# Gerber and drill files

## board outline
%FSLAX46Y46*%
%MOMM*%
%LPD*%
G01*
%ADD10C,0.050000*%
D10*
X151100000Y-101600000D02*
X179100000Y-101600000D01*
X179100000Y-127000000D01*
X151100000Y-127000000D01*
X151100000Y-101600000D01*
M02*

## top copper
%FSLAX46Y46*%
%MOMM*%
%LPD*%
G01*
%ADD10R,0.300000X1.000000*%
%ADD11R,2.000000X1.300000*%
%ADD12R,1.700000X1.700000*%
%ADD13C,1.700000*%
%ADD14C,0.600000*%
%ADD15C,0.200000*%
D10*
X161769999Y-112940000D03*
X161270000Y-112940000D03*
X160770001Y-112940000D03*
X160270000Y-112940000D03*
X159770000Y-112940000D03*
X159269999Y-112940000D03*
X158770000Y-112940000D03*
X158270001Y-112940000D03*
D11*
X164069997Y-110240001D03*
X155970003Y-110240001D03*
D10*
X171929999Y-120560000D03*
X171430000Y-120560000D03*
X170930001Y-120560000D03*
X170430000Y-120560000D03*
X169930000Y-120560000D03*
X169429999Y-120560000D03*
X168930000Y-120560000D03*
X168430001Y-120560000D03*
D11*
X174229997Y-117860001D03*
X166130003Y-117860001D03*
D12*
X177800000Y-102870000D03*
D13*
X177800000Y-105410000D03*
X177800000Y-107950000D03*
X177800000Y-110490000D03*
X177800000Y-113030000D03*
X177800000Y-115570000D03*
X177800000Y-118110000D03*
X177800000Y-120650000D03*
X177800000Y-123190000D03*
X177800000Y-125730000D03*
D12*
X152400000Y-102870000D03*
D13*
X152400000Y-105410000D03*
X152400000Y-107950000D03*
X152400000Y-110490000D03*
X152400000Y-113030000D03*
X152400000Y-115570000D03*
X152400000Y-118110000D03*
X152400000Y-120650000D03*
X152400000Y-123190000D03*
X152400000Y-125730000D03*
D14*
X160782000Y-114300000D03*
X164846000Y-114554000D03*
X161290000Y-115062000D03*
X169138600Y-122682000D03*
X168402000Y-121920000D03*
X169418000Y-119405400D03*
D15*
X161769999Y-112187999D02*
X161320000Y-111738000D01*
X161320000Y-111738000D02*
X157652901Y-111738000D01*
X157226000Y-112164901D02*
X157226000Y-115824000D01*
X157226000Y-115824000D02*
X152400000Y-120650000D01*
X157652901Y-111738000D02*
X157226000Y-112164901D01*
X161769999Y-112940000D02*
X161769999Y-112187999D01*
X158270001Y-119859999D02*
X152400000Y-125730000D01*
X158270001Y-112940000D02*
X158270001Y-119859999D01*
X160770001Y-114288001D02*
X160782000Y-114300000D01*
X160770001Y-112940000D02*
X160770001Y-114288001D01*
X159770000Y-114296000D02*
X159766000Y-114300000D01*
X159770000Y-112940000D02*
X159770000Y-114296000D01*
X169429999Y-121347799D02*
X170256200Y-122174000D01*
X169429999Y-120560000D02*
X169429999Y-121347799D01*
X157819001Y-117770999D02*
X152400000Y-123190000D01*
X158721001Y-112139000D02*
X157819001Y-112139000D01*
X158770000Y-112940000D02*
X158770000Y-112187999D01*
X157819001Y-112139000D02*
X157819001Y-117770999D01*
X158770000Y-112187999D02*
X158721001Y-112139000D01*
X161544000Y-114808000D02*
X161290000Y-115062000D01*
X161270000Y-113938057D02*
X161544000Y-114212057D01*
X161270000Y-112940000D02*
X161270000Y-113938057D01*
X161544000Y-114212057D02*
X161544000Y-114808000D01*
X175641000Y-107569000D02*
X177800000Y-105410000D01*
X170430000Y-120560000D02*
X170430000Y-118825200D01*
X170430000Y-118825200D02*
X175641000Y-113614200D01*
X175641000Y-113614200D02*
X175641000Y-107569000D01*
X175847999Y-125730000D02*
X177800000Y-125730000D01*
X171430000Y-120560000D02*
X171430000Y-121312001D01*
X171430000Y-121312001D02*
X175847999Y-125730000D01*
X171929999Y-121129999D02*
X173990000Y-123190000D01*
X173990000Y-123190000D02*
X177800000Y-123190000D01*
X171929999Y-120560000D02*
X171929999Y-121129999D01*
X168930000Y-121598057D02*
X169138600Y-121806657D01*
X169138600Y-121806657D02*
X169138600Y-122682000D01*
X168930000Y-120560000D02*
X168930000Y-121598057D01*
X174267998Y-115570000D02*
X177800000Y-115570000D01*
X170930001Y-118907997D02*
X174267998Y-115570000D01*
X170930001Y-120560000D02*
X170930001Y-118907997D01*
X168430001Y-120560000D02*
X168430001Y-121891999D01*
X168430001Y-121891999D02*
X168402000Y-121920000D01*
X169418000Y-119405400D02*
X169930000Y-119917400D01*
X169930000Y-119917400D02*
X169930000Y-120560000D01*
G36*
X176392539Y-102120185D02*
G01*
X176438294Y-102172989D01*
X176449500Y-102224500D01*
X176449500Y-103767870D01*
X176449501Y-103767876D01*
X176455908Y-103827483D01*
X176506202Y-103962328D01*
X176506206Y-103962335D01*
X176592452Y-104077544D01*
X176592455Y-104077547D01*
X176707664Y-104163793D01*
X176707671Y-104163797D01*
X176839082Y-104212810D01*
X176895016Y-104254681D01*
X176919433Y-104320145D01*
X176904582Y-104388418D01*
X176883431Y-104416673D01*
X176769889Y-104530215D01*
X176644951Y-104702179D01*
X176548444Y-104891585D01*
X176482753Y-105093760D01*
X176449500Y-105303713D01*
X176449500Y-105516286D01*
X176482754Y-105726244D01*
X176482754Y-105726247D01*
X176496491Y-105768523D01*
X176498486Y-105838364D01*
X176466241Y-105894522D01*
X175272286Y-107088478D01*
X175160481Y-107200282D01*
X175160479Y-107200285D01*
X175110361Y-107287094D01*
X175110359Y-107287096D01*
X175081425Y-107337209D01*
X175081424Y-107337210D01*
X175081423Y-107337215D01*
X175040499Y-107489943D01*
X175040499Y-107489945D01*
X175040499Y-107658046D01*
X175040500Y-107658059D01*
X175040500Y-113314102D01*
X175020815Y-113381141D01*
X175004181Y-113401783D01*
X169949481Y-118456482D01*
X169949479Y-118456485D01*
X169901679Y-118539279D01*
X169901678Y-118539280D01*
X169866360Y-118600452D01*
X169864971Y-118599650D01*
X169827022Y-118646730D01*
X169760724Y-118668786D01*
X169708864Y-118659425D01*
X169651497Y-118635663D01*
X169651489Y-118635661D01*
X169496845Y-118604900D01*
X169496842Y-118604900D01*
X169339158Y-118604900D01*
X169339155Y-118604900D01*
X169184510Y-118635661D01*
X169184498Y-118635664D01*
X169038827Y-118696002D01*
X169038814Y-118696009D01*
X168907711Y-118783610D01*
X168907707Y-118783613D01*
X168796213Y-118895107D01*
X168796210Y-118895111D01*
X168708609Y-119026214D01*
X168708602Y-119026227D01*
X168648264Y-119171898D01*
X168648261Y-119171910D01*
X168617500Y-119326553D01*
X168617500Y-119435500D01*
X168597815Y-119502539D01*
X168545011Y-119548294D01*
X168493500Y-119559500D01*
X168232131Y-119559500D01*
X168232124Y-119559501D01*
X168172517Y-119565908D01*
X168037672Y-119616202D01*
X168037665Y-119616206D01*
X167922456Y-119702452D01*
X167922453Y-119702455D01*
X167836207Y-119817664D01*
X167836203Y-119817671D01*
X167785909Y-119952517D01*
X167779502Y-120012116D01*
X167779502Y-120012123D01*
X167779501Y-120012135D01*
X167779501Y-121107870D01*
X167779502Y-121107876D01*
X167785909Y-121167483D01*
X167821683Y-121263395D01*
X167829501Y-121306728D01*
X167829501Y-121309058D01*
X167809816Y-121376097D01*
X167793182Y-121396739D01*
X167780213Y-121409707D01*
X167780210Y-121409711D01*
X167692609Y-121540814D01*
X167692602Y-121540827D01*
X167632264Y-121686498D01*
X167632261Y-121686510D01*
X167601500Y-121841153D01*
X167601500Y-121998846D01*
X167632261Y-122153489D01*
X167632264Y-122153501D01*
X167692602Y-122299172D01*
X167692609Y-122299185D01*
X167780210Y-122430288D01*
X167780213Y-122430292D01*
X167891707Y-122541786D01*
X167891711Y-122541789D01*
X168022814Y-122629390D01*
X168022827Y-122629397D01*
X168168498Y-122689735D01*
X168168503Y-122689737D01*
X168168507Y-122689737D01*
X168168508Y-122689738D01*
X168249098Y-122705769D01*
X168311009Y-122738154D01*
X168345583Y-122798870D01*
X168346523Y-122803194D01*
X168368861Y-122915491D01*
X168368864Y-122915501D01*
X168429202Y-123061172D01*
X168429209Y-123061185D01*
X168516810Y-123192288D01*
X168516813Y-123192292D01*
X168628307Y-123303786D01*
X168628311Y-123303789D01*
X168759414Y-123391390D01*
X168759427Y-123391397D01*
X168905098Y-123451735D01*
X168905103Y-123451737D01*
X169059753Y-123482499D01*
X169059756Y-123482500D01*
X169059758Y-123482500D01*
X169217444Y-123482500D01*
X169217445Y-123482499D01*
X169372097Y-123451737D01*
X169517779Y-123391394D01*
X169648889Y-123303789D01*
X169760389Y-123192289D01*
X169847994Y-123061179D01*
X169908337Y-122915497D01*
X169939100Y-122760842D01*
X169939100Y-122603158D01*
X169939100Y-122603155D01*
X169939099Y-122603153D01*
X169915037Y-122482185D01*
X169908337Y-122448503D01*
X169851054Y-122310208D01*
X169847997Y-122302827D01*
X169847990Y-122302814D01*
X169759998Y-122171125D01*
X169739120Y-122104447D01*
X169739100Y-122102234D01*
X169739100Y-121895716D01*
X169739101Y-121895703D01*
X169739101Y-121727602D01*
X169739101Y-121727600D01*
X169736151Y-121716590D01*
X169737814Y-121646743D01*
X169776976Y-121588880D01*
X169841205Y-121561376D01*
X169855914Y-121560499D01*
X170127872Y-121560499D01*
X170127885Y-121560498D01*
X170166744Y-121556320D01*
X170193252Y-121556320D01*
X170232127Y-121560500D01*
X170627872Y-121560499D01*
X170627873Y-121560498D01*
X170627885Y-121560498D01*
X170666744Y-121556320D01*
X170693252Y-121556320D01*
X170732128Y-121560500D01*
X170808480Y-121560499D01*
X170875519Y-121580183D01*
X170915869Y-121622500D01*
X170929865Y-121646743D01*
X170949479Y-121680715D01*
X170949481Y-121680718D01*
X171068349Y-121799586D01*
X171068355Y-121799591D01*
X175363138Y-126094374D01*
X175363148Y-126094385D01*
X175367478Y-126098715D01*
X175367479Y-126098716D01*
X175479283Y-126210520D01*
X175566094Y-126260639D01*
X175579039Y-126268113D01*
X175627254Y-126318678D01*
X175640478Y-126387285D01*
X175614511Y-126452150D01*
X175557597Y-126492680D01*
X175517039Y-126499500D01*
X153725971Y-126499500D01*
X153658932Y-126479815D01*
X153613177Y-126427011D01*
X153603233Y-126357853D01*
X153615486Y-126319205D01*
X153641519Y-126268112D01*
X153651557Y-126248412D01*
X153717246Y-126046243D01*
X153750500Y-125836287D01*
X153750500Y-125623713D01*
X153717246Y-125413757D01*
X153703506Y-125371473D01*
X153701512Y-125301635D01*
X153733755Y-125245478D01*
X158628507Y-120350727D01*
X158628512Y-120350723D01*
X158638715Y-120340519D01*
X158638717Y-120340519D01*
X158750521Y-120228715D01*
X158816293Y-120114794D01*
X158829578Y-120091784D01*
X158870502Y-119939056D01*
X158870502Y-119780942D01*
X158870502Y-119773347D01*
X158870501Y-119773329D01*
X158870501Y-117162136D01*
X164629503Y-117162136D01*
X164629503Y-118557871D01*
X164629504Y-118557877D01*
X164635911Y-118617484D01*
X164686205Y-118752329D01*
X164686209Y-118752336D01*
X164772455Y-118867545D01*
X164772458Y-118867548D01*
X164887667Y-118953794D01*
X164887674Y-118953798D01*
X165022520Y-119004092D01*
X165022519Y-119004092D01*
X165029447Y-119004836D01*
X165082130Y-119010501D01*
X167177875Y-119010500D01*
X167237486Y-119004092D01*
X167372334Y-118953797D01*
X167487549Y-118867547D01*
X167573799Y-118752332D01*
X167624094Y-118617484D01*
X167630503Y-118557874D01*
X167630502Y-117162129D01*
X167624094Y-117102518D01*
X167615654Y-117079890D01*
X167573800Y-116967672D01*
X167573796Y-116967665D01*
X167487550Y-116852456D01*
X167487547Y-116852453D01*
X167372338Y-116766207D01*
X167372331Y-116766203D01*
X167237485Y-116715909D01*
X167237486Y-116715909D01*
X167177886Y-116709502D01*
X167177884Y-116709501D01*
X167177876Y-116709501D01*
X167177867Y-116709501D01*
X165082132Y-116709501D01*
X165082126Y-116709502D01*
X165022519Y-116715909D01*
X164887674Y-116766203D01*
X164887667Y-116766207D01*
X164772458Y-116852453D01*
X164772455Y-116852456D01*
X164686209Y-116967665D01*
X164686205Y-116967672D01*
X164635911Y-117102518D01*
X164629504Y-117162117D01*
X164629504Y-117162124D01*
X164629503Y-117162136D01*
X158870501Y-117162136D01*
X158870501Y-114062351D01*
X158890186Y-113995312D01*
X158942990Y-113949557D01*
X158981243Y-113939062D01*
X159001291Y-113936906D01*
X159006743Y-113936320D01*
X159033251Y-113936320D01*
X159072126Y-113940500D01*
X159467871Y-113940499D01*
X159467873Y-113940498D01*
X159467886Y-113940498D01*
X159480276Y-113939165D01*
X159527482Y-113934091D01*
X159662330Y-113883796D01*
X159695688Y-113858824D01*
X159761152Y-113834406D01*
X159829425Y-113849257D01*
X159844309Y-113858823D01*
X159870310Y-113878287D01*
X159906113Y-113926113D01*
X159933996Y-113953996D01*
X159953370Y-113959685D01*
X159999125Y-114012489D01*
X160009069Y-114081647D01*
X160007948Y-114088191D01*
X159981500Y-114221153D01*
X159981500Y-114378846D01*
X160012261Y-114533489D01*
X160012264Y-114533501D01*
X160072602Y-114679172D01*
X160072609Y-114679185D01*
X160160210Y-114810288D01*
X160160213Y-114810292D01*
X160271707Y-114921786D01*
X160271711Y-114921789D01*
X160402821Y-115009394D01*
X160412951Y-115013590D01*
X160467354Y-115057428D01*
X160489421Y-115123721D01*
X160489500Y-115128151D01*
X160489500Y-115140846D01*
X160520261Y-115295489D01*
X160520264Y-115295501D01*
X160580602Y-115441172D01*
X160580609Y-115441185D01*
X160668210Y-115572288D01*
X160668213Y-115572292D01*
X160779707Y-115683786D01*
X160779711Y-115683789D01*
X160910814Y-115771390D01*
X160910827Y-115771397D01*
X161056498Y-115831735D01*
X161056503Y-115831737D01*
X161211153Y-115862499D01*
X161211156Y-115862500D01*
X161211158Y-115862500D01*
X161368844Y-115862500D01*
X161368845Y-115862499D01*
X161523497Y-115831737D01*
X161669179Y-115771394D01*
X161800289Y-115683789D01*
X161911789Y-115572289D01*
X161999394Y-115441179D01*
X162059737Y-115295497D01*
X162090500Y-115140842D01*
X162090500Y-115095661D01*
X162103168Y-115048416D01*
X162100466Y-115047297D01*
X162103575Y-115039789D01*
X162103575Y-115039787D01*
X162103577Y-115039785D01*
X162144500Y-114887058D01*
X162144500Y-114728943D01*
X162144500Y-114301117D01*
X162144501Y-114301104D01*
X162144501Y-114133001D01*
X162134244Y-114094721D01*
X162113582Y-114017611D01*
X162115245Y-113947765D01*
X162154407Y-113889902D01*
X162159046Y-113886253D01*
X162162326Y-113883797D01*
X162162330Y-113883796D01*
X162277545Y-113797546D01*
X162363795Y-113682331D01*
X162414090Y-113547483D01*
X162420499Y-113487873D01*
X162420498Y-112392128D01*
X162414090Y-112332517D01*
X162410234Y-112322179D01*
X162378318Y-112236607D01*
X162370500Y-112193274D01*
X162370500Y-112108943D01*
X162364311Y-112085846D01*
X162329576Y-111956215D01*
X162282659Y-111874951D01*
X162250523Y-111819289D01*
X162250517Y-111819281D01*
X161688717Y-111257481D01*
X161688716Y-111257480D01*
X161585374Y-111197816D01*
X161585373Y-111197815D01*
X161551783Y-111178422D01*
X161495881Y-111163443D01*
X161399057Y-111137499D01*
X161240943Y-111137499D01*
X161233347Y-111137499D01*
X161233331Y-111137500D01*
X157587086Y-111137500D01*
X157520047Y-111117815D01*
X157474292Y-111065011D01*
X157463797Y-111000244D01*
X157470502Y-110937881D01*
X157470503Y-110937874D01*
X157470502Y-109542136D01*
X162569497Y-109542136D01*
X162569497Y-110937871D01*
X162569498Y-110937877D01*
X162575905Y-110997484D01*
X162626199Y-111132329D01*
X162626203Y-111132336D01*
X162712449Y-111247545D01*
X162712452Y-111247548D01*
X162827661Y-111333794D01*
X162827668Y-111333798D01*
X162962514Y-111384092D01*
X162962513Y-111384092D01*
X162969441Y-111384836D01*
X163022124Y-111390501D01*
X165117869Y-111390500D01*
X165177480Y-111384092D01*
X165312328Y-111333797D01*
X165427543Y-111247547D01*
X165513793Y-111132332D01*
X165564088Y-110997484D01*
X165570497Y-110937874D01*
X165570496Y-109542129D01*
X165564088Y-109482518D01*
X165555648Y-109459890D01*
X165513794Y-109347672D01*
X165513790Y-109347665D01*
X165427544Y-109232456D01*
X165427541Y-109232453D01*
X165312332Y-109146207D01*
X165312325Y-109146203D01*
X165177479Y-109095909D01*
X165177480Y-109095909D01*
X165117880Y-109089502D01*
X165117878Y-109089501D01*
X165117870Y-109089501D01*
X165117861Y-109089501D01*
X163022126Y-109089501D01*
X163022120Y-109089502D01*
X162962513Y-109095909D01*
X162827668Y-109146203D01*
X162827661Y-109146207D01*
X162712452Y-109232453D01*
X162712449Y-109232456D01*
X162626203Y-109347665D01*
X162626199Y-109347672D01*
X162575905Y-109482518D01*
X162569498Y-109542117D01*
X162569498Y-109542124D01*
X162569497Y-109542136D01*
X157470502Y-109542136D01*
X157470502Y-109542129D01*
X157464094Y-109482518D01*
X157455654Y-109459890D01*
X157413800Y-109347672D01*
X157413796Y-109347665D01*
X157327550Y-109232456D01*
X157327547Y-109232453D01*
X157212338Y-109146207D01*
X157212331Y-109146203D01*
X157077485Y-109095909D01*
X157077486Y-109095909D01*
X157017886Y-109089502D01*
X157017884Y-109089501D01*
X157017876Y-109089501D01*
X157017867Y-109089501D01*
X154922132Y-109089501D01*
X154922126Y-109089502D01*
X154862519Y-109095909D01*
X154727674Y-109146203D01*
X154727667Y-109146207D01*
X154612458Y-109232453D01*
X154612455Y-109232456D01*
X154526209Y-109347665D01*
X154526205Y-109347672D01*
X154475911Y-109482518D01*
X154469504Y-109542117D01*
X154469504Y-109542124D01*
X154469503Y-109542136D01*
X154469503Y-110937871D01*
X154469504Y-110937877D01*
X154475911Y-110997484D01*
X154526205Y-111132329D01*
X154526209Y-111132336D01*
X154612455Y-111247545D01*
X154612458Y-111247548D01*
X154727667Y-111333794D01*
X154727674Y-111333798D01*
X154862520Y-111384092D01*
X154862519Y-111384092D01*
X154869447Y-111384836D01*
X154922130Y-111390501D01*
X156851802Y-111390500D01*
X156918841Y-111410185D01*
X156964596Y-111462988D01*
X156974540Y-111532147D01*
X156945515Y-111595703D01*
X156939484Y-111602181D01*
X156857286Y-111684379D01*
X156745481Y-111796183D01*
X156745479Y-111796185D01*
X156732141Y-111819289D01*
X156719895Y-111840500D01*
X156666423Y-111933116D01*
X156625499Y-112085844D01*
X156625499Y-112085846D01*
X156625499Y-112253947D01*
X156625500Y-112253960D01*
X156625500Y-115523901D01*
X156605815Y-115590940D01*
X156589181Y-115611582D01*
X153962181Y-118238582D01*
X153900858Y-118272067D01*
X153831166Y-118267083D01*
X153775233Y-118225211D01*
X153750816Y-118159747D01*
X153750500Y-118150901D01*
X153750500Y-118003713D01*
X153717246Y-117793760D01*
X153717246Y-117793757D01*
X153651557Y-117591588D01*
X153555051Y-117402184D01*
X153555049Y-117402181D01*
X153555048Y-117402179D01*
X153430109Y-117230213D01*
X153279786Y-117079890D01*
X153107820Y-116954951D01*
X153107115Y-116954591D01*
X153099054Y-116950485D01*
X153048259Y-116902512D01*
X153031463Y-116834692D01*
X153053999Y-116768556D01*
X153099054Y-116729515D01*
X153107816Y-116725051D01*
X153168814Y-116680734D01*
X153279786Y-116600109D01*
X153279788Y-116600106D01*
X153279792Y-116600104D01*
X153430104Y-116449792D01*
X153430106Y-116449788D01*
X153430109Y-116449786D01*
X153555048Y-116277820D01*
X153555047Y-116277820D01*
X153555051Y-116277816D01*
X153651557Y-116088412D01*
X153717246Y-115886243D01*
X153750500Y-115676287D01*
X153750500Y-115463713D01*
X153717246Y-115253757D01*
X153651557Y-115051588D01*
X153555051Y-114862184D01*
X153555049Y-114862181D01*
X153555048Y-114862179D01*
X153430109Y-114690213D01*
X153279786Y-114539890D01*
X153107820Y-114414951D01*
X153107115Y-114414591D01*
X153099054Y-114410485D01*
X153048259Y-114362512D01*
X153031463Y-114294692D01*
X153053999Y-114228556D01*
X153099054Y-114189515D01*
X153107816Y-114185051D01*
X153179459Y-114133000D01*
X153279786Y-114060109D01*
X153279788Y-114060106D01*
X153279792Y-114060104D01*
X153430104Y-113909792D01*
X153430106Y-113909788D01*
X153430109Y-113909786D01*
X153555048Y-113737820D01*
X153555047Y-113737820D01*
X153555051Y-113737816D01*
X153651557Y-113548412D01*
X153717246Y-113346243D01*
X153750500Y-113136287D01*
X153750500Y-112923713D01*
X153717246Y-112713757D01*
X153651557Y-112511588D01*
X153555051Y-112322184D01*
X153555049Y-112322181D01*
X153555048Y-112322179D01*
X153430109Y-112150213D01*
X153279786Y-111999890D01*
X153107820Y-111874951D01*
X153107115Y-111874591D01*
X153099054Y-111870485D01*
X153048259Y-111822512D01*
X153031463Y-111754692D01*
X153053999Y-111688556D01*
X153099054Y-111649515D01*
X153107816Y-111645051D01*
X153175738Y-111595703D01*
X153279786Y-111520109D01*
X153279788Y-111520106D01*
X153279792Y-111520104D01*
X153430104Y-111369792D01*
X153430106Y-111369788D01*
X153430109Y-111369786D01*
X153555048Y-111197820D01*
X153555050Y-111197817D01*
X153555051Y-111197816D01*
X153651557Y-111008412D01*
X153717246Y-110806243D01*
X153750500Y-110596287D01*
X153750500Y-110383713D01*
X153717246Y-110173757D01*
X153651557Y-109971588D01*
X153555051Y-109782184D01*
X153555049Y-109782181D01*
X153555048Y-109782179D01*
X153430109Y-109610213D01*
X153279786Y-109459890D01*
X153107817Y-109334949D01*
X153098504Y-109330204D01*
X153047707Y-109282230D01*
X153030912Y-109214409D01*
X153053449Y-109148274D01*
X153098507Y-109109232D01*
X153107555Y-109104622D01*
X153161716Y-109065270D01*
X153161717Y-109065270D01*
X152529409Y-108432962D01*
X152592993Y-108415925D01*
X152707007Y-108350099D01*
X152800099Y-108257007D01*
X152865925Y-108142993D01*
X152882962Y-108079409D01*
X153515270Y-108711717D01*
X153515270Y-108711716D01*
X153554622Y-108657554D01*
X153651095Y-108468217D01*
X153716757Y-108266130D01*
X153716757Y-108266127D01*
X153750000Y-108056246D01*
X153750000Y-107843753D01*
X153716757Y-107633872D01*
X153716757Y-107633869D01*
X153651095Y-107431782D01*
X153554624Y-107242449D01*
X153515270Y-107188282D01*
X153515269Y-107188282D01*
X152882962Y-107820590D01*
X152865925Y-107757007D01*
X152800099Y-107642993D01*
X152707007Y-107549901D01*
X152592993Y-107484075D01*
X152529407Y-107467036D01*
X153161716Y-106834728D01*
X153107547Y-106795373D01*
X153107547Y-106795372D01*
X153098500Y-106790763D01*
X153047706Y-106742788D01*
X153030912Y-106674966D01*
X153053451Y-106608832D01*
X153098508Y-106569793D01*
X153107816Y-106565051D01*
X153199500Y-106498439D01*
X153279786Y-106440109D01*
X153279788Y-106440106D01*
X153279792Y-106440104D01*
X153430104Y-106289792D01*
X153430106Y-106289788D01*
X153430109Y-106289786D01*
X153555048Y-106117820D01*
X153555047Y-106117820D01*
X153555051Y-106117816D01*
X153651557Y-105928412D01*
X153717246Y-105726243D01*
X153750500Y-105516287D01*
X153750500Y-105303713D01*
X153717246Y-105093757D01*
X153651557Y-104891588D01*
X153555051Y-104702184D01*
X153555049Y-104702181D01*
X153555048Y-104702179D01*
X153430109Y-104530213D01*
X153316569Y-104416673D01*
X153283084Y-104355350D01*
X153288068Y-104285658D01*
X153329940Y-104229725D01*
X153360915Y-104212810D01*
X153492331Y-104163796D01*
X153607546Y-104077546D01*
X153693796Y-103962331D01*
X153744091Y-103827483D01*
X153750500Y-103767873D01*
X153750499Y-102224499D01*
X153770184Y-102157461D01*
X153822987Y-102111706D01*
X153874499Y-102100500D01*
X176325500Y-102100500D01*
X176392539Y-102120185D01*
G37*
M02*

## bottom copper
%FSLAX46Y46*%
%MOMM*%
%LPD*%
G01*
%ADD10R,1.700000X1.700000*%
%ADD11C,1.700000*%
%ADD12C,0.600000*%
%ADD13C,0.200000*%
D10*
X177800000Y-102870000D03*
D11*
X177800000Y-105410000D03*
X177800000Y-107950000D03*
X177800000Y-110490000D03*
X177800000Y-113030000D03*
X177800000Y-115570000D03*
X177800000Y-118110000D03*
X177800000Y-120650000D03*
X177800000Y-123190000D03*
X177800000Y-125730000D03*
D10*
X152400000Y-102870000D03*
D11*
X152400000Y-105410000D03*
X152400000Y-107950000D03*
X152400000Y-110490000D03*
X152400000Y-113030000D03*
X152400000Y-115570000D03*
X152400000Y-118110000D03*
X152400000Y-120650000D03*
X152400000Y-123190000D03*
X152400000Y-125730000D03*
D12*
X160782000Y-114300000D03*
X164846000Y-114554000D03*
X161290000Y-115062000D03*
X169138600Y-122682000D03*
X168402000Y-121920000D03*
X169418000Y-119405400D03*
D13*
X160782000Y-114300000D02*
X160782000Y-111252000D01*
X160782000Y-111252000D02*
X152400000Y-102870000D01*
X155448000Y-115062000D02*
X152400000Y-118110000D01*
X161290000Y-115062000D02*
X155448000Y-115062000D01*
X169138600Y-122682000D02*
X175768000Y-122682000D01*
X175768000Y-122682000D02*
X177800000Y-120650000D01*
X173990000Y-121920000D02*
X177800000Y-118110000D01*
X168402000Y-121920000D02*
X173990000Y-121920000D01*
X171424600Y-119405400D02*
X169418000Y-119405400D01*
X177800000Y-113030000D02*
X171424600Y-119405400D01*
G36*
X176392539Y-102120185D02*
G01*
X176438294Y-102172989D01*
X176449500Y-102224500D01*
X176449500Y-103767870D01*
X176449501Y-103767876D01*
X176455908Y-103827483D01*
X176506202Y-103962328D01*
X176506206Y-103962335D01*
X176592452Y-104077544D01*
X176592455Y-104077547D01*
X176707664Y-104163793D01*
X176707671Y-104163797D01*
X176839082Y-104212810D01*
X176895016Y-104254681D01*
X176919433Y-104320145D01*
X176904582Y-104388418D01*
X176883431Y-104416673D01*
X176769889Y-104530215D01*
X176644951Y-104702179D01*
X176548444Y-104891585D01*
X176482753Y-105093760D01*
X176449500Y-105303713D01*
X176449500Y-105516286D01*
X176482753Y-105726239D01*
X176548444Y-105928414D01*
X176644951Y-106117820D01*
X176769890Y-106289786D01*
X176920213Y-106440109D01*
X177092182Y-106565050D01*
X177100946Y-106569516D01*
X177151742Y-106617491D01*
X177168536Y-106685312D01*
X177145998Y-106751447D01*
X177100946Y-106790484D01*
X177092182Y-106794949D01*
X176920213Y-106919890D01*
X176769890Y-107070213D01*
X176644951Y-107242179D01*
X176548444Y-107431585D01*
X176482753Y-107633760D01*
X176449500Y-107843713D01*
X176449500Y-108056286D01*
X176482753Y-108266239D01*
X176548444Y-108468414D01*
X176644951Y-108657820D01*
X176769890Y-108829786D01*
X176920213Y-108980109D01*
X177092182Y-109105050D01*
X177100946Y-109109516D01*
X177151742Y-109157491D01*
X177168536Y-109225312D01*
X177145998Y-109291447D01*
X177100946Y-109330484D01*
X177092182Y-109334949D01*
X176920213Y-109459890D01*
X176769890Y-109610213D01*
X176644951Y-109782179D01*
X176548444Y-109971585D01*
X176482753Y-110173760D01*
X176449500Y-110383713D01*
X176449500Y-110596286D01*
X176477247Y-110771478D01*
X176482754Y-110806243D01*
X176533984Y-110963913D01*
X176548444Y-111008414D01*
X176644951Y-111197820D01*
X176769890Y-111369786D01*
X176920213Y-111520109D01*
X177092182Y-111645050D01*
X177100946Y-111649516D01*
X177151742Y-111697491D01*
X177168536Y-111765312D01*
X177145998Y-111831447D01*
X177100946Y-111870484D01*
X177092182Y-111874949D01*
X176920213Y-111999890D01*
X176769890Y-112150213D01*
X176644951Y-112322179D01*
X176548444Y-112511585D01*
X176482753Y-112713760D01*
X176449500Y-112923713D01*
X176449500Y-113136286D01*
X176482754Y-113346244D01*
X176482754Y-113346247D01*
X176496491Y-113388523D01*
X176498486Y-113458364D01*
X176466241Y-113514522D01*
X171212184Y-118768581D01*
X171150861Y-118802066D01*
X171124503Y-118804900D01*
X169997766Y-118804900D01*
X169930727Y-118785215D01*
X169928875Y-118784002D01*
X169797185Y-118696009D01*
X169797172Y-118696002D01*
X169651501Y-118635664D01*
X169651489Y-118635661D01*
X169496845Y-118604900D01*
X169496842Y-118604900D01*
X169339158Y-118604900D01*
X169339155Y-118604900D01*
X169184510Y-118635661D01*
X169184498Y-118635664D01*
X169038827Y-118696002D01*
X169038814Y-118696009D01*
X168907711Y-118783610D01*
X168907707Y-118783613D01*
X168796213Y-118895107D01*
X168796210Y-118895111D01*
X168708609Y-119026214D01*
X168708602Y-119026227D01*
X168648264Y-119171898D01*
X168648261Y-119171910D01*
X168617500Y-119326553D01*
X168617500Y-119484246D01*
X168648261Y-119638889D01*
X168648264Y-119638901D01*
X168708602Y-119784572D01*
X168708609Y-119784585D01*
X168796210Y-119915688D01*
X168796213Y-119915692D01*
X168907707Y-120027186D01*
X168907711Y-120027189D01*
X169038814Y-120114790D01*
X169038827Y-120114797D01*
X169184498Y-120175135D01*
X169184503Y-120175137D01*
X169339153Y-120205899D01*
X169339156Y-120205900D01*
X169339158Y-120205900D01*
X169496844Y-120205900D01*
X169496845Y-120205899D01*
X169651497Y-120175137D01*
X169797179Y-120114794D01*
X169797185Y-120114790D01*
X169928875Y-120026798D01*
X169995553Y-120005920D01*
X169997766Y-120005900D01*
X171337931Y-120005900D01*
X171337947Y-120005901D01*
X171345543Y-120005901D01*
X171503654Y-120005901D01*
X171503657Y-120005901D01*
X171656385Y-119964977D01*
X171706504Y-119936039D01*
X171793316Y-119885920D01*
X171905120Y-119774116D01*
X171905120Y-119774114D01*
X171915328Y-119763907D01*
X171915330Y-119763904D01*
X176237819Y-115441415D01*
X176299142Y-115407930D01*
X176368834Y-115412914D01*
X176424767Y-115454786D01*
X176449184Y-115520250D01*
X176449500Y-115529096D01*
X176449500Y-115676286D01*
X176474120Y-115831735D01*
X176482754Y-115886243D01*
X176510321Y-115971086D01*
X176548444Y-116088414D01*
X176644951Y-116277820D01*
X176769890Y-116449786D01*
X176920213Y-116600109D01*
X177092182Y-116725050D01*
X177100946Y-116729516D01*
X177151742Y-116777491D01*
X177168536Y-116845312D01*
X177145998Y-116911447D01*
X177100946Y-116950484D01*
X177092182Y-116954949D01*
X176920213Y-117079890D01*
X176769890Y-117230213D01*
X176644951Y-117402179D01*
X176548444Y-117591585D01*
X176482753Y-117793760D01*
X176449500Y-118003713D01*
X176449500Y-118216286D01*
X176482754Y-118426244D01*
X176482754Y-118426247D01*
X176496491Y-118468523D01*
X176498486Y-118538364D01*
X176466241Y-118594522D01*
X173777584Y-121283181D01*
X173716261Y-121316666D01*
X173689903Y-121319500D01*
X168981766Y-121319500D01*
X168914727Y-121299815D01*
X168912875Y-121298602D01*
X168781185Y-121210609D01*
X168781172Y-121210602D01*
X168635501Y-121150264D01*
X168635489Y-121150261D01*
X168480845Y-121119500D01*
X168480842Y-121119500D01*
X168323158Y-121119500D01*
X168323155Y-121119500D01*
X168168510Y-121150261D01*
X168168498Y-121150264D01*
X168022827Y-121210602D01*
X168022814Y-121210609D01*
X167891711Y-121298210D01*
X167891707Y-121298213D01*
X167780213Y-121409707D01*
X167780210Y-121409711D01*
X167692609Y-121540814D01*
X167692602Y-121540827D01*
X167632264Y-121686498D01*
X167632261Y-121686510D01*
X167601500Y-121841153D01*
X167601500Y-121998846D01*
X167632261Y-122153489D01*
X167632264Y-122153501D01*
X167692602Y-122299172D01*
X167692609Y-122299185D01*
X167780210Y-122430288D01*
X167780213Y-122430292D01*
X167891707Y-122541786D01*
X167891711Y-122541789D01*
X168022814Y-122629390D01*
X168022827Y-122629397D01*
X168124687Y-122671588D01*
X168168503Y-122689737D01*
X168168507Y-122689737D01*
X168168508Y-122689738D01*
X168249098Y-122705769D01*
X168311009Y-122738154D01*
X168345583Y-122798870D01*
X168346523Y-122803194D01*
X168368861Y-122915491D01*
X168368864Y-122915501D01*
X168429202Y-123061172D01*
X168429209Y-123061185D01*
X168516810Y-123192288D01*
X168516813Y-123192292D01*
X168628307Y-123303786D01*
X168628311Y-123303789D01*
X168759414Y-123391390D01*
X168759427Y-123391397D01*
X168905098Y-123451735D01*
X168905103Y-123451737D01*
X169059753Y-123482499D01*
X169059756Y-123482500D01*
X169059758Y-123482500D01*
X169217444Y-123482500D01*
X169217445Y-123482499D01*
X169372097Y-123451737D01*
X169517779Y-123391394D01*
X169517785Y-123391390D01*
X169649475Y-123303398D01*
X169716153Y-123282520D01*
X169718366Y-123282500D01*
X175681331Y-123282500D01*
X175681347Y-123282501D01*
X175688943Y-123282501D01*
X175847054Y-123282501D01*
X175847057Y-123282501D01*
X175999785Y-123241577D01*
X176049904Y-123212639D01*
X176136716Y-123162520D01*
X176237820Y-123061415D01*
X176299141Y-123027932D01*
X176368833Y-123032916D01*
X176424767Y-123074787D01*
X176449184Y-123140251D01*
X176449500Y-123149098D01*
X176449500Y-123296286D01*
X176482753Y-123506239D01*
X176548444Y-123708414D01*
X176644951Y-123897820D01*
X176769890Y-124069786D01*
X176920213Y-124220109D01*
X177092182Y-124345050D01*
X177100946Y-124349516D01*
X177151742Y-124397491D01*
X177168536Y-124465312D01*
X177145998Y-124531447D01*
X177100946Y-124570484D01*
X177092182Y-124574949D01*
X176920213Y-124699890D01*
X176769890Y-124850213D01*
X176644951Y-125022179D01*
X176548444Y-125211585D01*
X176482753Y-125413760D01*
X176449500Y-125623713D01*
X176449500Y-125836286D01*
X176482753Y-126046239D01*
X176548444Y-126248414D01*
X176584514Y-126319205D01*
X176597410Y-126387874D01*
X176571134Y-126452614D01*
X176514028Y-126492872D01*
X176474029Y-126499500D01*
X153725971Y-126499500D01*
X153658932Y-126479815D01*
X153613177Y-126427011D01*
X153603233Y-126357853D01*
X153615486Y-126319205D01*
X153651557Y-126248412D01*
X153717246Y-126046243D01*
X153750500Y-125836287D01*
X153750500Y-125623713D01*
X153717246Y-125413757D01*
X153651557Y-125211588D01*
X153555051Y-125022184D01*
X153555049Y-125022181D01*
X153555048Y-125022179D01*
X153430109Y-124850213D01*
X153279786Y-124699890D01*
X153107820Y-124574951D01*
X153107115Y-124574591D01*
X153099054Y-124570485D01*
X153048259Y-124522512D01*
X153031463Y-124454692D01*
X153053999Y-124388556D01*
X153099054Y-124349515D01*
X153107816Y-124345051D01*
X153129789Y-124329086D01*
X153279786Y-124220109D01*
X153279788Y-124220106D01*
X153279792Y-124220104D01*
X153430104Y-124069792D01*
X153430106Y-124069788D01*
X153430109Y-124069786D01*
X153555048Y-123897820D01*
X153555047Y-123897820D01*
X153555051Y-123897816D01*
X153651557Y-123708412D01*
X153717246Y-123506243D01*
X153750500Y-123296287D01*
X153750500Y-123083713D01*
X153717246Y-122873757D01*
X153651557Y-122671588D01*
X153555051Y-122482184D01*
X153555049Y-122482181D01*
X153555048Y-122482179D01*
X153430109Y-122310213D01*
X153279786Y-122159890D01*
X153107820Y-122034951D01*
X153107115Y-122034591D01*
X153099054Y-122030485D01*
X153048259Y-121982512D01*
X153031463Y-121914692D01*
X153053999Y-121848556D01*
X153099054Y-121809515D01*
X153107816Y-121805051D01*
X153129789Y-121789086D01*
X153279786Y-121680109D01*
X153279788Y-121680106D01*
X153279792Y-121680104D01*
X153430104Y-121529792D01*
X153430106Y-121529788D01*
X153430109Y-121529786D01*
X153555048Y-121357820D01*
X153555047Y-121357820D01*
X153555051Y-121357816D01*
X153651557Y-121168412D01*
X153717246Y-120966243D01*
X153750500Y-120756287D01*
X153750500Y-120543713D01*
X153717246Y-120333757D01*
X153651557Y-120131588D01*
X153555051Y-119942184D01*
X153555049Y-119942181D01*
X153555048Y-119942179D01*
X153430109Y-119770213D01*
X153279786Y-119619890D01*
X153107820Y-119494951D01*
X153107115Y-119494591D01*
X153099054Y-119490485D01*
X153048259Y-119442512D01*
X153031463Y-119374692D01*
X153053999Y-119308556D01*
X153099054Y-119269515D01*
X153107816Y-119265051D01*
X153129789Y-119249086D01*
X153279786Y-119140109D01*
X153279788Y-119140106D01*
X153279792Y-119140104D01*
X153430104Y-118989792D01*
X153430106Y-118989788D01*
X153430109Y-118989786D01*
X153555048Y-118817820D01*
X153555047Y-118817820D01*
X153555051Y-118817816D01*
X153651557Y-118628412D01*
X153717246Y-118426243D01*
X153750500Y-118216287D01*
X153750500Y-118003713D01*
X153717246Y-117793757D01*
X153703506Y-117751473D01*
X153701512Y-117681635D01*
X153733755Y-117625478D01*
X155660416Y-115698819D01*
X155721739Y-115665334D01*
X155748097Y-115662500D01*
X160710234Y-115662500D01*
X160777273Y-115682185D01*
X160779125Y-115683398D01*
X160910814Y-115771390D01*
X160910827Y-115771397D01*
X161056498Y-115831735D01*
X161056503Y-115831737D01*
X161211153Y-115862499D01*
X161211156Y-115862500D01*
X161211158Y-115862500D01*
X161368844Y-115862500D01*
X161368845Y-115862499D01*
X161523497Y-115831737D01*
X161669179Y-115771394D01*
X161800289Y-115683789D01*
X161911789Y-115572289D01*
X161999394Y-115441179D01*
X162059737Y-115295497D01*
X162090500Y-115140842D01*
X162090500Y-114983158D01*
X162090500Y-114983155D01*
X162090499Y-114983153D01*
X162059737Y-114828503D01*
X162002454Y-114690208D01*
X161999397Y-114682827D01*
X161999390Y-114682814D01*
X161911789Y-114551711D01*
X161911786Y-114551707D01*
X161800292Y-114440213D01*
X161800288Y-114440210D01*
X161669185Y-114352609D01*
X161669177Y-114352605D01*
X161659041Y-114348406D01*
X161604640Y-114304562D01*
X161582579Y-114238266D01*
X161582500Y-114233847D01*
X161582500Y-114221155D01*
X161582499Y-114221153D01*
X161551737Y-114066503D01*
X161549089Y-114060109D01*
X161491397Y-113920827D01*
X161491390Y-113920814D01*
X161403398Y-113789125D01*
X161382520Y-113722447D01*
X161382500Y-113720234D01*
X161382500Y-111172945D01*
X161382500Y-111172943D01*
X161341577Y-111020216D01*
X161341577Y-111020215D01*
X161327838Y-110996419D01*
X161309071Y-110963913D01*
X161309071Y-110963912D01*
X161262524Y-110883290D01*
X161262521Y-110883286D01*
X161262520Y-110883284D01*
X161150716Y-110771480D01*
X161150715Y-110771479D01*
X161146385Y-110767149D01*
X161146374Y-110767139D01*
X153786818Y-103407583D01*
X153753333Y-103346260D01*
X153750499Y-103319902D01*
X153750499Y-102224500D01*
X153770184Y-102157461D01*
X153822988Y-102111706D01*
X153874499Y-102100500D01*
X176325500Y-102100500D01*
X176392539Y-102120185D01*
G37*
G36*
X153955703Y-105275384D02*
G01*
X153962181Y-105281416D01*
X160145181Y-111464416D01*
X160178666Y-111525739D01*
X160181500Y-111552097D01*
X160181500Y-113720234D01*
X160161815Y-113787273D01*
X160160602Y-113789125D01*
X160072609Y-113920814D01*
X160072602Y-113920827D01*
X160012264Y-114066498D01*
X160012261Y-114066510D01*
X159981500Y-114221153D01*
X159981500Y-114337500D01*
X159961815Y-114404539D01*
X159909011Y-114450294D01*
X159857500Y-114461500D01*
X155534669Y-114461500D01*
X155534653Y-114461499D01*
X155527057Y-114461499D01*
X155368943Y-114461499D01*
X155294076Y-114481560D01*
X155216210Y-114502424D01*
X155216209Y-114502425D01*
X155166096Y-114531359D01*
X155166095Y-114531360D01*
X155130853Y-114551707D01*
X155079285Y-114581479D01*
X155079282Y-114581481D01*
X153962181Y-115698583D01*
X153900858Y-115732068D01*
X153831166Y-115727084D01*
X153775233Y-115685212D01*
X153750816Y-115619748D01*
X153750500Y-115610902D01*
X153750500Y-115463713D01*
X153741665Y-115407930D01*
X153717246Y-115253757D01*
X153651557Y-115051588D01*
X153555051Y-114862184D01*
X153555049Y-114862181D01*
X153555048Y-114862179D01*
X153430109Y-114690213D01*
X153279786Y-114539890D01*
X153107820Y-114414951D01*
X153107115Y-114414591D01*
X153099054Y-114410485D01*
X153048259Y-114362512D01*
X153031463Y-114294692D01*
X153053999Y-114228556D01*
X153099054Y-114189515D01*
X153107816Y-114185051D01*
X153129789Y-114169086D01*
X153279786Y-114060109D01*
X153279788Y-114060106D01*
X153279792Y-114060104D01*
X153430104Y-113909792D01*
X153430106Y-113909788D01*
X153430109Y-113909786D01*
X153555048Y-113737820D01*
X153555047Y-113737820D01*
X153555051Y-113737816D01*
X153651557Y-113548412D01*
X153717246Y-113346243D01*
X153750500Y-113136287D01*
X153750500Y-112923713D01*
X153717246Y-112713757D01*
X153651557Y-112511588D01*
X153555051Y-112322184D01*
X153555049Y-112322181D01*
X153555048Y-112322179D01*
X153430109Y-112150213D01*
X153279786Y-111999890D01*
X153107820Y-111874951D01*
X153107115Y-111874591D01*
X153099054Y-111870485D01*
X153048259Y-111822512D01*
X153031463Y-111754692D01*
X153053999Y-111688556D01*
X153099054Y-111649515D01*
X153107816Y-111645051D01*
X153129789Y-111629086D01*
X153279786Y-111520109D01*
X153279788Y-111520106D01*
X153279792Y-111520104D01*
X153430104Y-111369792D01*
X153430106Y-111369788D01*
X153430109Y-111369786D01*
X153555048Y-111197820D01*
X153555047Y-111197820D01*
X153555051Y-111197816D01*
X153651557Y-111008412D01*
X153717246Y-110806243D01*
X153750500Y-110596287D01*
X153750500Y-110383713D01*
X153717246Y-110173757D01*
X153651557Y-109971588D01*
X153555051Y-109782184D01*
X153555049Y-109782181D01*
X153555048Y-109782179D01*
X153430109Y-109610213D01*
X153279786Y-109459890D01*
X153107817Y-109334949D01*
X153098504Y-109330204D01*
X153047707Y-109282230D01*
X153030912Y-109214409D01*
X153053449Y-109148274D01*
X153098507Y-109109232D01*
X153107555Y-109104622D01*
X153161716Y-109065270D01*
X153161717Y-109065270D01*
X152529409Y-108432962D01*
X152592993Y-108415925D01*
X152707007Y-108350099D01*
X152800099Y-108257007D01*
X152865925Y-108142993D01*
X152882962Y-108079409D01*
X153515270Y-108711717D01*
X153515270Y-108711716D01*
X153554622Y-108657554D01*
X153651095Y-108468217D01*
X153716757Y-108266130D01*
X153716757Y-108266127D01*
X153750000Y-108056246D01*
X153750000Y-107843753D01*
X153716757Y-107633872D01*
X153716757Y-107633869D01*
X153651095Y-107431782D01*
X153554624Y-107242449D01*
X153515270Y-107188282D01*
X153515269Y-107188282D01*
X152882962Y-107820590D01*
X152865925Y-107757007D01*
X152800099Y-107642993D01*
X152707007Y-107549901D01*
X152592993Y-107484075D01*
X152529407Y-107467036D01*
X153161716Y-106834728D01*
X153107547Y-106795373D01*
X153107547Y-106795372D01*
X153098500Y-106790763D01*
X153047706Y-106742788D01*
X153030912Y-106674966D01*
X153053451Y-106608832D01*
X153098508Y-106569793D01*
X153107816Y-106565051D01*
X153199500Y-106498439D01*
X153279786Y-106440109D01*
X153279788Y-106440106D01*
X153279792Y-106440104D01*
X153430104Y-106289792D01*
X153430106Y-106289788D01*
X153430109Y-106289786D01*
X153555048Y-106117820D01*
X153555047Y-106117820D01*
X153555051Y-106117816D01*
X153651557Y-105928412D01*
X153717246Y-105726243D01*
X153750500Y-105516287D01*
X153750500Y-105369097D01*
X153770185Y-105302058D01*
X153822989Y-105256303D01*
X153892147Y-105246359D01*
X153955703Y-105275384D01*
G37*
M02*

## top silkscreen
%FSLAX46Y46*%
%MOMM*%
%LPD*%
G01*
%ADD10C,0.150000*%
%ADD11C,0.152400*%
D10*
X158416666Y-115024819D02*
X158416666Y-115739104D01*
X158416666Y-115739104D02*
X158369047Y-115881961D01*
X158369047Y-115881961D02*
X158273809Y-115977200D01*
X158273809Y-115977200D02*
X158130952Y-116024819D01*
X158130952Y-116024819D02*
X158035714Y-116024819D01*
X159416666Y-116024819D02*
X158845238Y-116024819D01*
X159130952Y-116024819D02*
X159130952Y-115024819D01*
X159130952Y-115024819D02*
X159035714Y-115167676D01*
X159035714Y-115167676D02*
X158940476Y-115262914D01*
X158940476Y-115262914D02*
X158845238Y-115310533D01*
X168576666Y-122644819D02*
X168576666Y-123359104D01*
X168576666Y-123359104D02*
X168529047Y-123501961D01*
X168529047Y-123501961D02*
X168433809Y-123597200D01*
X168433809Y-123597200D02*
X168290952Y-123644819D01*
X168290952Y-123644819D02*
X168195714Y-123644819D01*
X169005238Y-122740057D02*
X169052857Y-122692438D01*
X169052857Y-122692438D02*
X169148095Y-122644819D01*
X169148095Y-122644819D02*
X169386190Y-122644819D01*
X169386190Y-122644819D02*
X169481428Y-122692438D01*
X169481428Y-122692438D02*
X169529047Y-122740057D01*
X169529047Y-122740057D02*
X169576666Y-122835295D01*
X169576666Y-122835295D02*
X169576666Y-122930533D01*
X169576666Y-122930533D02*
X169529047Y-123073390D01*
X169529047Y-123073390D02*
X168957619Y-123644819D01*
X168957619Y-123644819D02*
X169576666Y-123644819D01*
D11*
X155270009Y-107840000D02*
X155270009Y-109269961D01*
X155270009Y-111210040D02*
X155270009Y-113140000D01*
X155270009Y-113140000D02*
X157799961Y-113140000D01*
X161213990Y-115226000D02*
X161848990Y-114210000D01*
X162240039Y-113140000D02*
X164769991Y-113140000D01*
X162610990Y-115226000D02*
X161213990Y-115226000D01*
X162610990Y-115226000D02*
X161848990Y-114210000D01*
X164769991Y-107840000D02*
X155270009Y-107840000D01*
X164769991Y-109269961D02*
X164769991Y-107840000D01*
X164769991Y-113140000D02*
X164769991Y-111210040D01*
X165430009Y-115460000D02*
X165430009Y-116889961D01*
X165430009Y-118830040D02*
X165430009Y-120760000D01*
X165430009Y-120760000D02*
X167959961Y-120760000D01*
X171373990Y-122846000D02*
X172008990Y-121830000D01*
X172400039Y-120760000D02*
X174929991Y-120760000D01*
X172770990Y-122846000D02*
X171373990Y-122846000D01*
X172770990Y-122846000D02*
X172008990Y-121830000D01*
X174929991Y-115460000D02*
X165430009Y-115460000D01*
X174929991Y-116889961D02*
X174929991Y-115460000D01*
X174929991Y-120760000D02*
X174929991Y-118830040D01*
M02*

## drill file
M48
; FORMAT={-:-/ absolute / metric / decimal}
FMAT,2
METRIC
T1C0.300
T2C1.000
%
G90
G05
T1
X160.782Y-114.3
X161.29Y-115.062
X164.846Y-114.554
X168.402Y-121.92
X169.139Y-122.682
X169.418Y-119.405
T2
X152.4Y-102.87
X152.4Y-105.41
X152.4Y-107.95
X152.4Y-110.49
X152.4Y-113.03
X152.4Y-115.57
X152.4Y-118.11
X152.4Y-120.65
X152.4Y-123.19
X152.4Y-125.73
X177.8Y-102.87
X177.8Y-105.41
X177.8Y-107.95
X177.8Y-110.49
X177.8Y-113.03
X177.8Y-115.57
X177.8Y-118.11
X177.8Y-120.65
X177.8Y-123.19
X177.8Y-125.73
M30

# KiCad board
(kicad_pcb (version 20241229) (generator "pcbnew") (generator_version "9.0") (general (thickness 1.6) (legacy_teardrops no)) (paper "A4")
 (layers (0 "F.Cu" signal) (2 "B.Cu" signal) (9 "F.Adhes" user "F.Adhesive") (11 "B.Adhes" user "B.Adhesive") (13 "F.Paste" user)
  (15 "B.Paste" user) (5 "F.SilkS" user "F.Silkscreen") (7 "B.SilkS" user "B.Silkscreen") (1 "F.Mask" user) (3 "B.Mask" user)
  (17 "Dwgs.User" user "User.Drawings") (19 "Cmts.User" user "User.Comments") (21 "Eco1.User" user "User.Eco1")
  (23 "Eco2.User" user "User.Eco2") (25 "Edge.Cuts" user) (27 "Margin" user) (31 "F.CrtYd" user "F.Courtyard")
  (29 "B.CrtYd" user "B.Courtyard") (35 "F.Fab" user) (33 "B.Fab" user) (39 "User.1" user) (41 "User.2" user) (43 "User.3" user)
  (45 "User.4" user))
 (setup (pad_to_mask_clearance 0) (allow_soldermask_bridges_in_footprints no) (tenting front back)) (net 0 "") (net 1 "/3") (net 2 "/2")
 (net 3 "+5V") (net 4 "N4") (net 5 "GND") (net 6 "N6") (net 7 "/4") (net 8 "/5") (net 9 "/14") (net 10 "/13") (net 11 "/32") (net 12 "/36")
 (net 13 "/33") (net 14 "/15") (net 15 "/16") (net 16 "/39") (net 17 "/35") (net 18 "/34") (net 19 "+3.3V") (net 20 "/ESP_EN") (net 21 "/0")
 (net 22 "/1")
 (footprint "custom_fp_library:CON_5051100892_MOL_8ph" (layer "F.Cu") (at 160.02 110.49 180)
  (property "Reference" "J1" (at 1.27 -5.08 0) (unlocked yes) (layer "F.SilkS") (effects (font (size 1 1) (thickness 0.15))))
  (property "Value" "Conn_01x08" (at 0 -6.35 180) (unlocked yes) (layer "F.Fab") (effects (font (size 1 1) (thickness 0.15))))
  (fp_line (start 4.749991 2.65) (end 4.749991 1.220039) (stroke (width 0.1524) (type solid)) (layer "F.SilkS"))
  (fp_line (start 4.749991 -0.72004) (end 4.749991 -2.65) (stroke (width 0.1524) (type solid)) (layer "F.SilkS"))
  (fp_line (start 4.749991 -2.65) (end 2.220039 -2.65) (stroke (width 0.1524) (type solid)) (layer "F.SilkS"))
  (fp_line (start -1.19399 -4.736) (end -1.82899 -3.72) (stroke (width 0.1524) (type solid)) (layer "F.SilkS"))
  (fp_line (start -2.220039 -2.65) (end -4.749991 -2.65) (stroke (width 0.1524) (type solid)) (layer "F.SilkS"))
  (fp_line (start -2.59099 -4.736) (end -1.19399 -4.736) (stroke (width 0.1524) (type solid)) (layer "F.SilkS"))
  (fp_line (start -2.59099 -4.736) (end -1.82899 -3.72) (stroke (width 0.1524) (type solid)) (layer "F.SilkS"))
  (fp_line (start -4.749991 2.65) (end 4.749991 2.65) (stroke (width 0.1524) (type solid)) (layer "F.SilkS"))
  (fp_line (start -4.749991 1.220039) (end -4.749991 2.65) (stroke (width 0.1524) (type solid)) (layer "F.SilkS"))
  (fp_line (start -4.749991 -2.65) (end -4.749991 -0.72004) (stroke (width 0.1524) (type solid)) (layer "F.SilkS"))
  (pad "1" smd rect (at -1.749999 -2.45 180) (size 0.3 1) (layers "F.Cu" "F.Mask" "F.Paste") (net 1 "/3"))
  (pad "2" smd rect (at -1.25 -2.45 180) (size 0.3 1) (layers "F.Cu" "F.Mask" "F.Paste") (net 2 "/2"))
  (pad "3" smd rect (at -0.750001 -2.45 180) (size 0.3 1) (layers "F.Cu" "F.Mask" "F.Paste") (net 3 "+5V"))
  (pad "4" smd rect (at -0.25 -2.45 180) (size 0.3 1) (layers "F.Cu" "F.Mask" "F.Paste") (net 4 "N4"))
  (pad "5" smd rect (at 0.25 -2.45 180) (size 0.3 1) (layers "F.Cu" "F.Mask" "F.Paste") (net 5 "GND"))
  (pad "6" smd rect (at 0.750001 -2.45 180) (size 0.3 1) (layers "F.Cu" "F.Mask" "F.Paste") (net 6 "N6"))
  (pad "7" smd rect (at 1.25 -2.45 180) (size 0.3 1) (layers "F.Cu" "F.Mask" "F.Paste") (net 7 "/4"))
  (pad "8" smd rect (at 1.749999 -2.45 180) (size 0.3 1) (layers "F.Cu" "F.Mask" "F.Paste") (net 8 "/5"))
  (pad "P1" smd rect (at -4.049997 0.249999 180) (size 2 1.3) (layers "F.Cu" "F.Mask" "F.Paste"))
  (pad "P2" smd rect (at 4.049997 0.249999 180) (size 2 1.3) (layers "F.Cu" "F.Mask" "F.Paste")))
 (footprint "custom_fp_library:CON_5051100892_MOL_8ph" (layer "F.Cu") (at 170.18 118.11 180)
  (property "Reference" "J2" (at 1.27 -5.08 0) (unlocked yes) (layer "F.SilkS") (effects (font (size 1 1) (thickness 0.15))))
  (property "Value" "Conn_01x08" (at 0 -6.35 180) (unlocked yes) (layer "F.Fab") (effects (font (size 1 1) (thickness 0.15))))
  (fp_line (start 4.749991 2.65) (end 4.749991 1.220039) (stroke (width 0.1524) (type solid)) (layer "F.SilkS"))
  (fp_line (start 4.749991 -0.72004) (end 4.749991 -2.65) (stroke (width 0.1524) (type solid)) (layer "F.SilkS"))
  (fp_line (start 4.749991 -2.65) (end 2.220039 -2.65) (stroke (width 0.1524) (type solid)) (layer "F.SilkS"))
  (fp_line (start -1.19399 -4.736) (end -1.82899 -3.72) (stroke (width 0.1524) (type solid)) (layer "F.SilkS"))
  (fp_line (start -2.220039 -2.65) (end -4.749991 -2.65) (stroke (width 0.1524) (type solid)) (layer "F.SilkS"))
  (fp_line (start -2.59099 -4.736) (end -1.19399 -4.736) (stroke (width 0.1524) (type solid)) (layer "F.SilkS"))
  (fp_line (start -2.59099 -4.736) (end -1.82899 -3.72) (stroke (width 0.1524) (type solid)) (layer "F.SilkS"))
  (fp_line (start -4.749991 2.65) (end 4.749991 2.65) (stroke (width 0.1524) (type solid)) (layer "F.SilkS"))
  (fp_line (start -4.749991 1.220039) (end -4.749991 2.65) (stroke (width 0.1524) (type solid)) (layer "F.SilkS"))
  (fp_line (start -4.749991 -2.65) (end -4.749991 -0.72004) (stroke (width 0.1524) (type solid)) (layer "F.SilkS"))
  (pad "1" smd rect (at -1.749999 -2.45 180) (size 0.3 1) (layers "F.Cu" "F.Mask" "F.Paste") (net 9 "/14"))
  (pad "2" smd rect (at -1.25 -2.45 180) (size 0.3 1) (layers "F.Cu" "F.Mask" "F.Paste") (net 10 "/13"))
  (pad "3" smd rect (at -0.750001 -2.45 180) (size 0.3 1) (layers "F.Cu" "F.Mask" "F.Paste") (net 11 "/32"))
  (pad "4" smd rect (at -0.25 -2.45 180) (size 0.3 1) (layers "F.Cu" "F.Mask" "F.Paste") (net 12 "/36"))
  (pad "5" smd rect (at 0.25 -2.45 180) (size 0.3 1) (layers "F.Cu" "F.Mask" "F.Paste") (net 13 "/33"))
  (pad "6" smd rect (at 0.750001 -2.45 180) (size 0.3 1) (layers "F.Cu" "F.Mask" "F.Paste") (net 5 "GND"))
  (pad "7" smd rect (at 1.25 -2.45 180) (size 0.3 1) (layers "F.Cu" "F.Mask" "F.Paste") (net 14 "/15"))
  (pad "8" smd rect (at 1.749999 -2.45 180) (size 0.3 1) (layers "F.Cu" "F.Mask" "F.Paste") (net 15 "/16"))
  (pad "P1" smd rect (at -4.049997 0.249999 180) (size 2 1.3) (layers "F.Cu" "F.Mask" "F.Paste"))
  (pad "P2" smd rect (at 4.049997 0.249999 180) (size 2 1.3) (layers "F.Cu" "F.Mask" "F.Paste")))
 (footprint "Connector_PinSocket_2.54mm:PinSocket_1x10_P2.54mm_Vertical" (layer "B.Cu") (at 177.8 102.87 180)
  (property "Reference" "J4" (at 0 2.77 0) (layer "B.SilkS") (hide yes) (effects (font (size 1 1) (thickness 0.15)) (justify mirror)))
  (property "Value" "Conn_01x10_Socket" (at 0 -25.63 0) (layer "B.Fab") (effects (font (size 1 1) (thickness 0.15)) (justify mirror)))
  (pad "1" thru_hole rect (at 0 0 180) (size 1.7 1.7) (drill 1) (layers "*.Cu" "*.Mask") (remove_unused_layers no) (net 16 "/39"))
  (pad "2" thru_hole circle (at 0 -2.54 180) (size 1.7 1.7) (drill 1) (layers "*.Cu" "*.Mask") (remove_unused_layers no) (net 12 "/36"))
  (pad "3" thru_hole circle (at 0 -5.08 180) (size 1.7 1.7) (drill 1) (layers "*.Cu" "*.Mask") (remove_unused_layers no) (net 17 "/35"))
  (pad "4" thru_hole circle (at 0 -7.62 180) (size 1.7 1.7) (drill 1) (layers "*.Cu" "*.Mask") (remove_unused_layers no) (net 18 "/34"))
  (pad "5" thru_hole circle (at 0 -10.16 180) (size 1.7 1.7) (drill 1) (layers "*.Cu" "*.Mask") (remove_unused_layers no) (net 13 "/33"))
  (pad "6" thru_hole circle (at 0 -12.7 180) (size 1.7 1.7) (drill 1) (layers "*.Cu" "*.Mask") (remove_unused_layers no) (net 11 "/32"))
  (pad "7" thru_hole circle (at 0 -15.24 180) (size 1.7 1.7) (drill 1) (layers "*.Cu" "*.Mask") (remove_unused_layers no) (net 15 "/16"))
  (pad "8" thru_hole circle (at 0 -17.78 180) (size 1.7 1.7) (drill 1) (layers "*.Cu" "*.Mask") (remove_unused_layers no) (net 14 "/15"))
  (pad "9" thru_hole circle (at 0 -20.32 180) (size 1.7 1.7) (drill 1) (layers "*.Cu" "*.Mask") (remove_unused_layers no) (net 9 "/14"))
  (pad "10" thru_hole circle (at 0 -22.86 180) (size 1.7 1.7) (drill 1) (layers "*.Cu" "*.Mask") (remove_unused_layers no) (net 10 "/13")))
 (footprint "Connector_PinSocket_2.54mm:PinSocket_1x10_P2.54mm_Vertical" (layer "B.Cu") (at 152.4 102.87 180)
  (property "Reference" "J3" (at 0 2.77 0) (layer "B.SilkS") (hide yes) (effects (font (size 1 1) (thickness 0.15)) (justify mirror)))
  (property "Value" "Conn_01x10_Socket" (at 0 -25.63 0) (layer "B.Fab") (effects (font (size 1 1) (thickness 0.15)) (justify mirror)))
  (pad "1" thru_hole rect (at 0 0 180) (size 1.7 1.7) (drill 1) (layers "*.Cu" "*.Mask") (remove_unused_layers no) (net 3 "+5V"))
  (pad "2" thru_hole circle (at 0 -2.54 180) (size 1.7 1.7) (drill 1) (layers "*.Cu" "*.Mask") (remove_unused_layers no) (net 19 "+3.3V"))
  (pad "3" thru_hole circle (at 0 -5.08 180) (size 1.7 1.7) (drill 1) (layers "*.Cu" "*.Mask") (remove_unused_layers no) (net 5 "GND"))
  (pad "4" thru_hole circle (at 0 -7.62 180) (size 1.7 1.7) (drill 1) (layers "*.Cu" "*.Mask") (remove_unused_layers no) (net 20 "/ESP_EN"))
  (pad "5" thru_hole circle (at 0 -10.16 180) (size 1.7 1.7) (drill 1) (layers "*.Cu" "*.Mask") (remove_unused_layers no) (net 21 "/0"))
  (pad "6" thru_hole circle (at 0 -12.7 180) (size 1.7 1.7) (drill 1) (layers "*.Cu" "*.Mask") (remove_unused_layers no) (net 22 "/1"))
  (pad "7" thru_hole circle (at 0 -15.24 180) (size 1.7 1.7) (drill 1) (layers "*.Cu" "*.Mask") (remove_unused_layers no) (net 2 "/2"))
  (pad "8" thru_hole circle (at 0 -17.78 180) (size 1.7 1.7) (drill 1) (layers "*.Cu" "*.Mask") (remove_unused_layers no) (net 1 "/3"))
  (pad "9" thru_hole circle (at 0 -20.32 180) (size 1.7 1.7) (drill 1) (layers "*.Cu" "*.Mask") (remove_unused_layers no) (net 7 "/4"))
  (pad "10" thru_hole circle (at 0 -22.86 180) (size 1.7 1.7) (drill 1) (layers "*.Cu" "*.Mask") (remove_unused_layers no) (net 8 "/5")))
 (gr_rect (start 151.1 101.6) (end 179.1 127) (stroke (width 0.05) (type solid)) (fill no) (layer "Edge.Cuts"))
 (segment (start 161.769999 112.187999) (end 161.32 111.738) (width 0.2) (layer "F.Cu") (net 1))
 (segment (start 161.32 111.738) (end 157.652901 111.738) (width 0.2) (layer "F.Cu") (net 1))
 (segment (start 157.226 112.164901) (end 157.226 115.824) (width 0.2) (layer "F.Cu") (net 1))
 (segment (start 157.226 115.824) (end 152.4 120.65) (width 0.2) (layer "F.Cu") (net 1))
 (segment (start 157.652901 111.738) (end 157.226 112.164901) (width 0.2) (layer "F.Cu") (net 1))
 (segment (start 161.769999 112.94) (end 161.769999 112.187999) (width 0.2) (layer "F.Cu") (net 1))
 (segment (start 158.270001 119.859999) (end 152.4 125.73) (width 0.2) (layer "F.Cu") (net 8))
 (segment (start 158.270001 112.94) (end 158.270001 119.859999) (width 0.2) (layer "F.Cu") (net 8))
 (segment (start 160.770001 114.288001) (end 160.782 114.3) (width 0.2) (layer "F.Cu") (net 3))
 (segment (start 160.770001 112.94) (end 160.770001 114.288001) (width 0.2) (layer "F.Cu") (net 3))
 (via (at 160.782 114.3) (size 0.6) (drill 0.3) (layers "F.Cu" "B.Cu") (free yes) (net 3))
 (segment (start 160.782 114.3) (end 160.782 111.252) (width 0.2) (layer "B.Cu") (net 3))
 (segment (start 160.782 111.252) (end 152.4 102.87) (width 0.2) (layer "B.Cu") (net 3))
 (segment (start 159.77 114.296) (end 159.766 114.3) (width 0.2) (layer "F.Cu") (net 5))
 (segment (start 159.77 112.94) (end 159.77 114.296) (width 0.2) (layer "F.Cu") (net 5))
 (segment (start 169.429999 121.347799) (end 170.2562 122.174) (width 0.2) (layer "F.Cu") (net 5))
 (segment (start 169.429999 120.56) (end 169.429999 121.347799) (width 0.2) (layer "F.Cu") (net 5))
 (via (at 164.846 114.554) (size 0.6) (drill 0.3) (layers "F.Cu" "B.Cu") (free yes) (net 5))
 (segment (start 157.819001 117.770999) (end 152.4 123.19) (width 0.2) (layer "F.Cu") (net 7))
 (segment (start 158.721001 112.139) (end 157.819001 112.139) (width 0.2) (layer "F.Cu") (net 7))
 (segment (start 158.77 112.94) (end 158.77 112.187999) (width 0.2) (layer "F.Cu") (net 7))
 (segment (start 157.819001 112.139) (end 157.819001 117.770999) (width 0.2) (layer "F.Cu") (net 7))
 (segment (start 158.77 112.187999) (end 158.721001 112.139) (width 0.2) (layer "F.Cu") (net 7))
 (segment (start 161.544 114.808) (end 161.29 115.062) (width 0.2) (layer "F.Cu") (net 2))
 (segment (start 161.27 113.938057) (end 161.544 114.212057) (width 0.2) (layer "F.Cu") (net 2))
 (segment (start 161.27 112.94) (end 161.27 113.938057) (width 0.2) (layer "F.Cu") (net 2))
 (segment (start 161.544 114.212057) (end 161.544 114.808) (width 0.2) (layer "F.Cu") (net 2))
 (via (at 161.29 115.062) (size 0.6) (drill 0.3) (layers "F.Cu" "B.Cu") (free yes) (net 2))
 (segment (start 155.448 115.062) (end 152.4 118.11) (width 0.2) (layer "B.Cu") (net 2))
 (segment (start 161.29 115.062) (end 155.448 115.062) (width 0.2) (layer "B.Cu") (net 2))
 (segment (start 175.641 107.569) (end 177.8 105.41) (width 0.2) (layer "F.Cu") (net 12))
 (segment (start 170.43 120.56) (end 170.43 118.8252) (width 0.2) (layer "F.Cu") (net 12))
 (segment (start 170.43 118.8252) (end 175.641 113.6142) (width 0.2) (layer "F.Cu") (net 12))
 (segment (start 175.641 113.6142) (end 175.641 107.569) (width 0.2) (layer "F.Cu") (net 12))
 (segment (start 175.847999 125.73) (end 177.8 125.73) (width 0.2) (layer "F.Cu") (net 10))
 (segment (start 171.43 120.56) (end 171.43 121.312001) (width 0.2) (layer "F.Cu") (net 10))
 (segment (start 171.43 121.312001) (end 175.847999 125.73) (width 0.2) (layer "F.Cu") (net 10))
 (segment (start 171.929999 121.129999) (end 173.99 123.19) (width 0.2) (layer "F.Cu") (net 9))
 (segment (start 173.99 123.19) (end 177.8 123.19) (width 0.2) (layer "F.Cu") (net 9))
 (segment (start 171.929999 120.56) (end 171.929999 121.129999) (width 0.2) (layer "F.Cu") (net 9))
 (segment (start 168.93 121.598057) (end 169.1386 121.806657) (width 0.2) (layer "F.Cu") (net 14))
 (segment (start 169.1386 121.806657) (end 169.1386 122.682) (width 0.2) (layer "F.Cu") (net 14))
 (segment (start 168.93 120.56) (end 168.93 121.598057) (width 0.2) (layer "F.Cu") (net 14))
 (via (at 169.1386 122.682) (size 0.6) (drill 0.3) (layers "F.Cu" "B.Cu") (free yes) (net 14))
 (segment (start 169.1386 122.682) (end 175.768 122.682) (width 0.2) (layer "B.Cu") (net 14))
 (segment (start 175.768 122.682) (end 177.8 120.65) (width 0.2) (layer "B.Cu") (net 14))
 (segment (start 174.267998 115.57) (end 177.8 115.57) (width 0.2) (layer "F.Cu") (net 11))
 (segment (start 170.930001 118.907997) (end 174.267998 115.57) (width 0.2) (layer "F.Cu") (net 11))
 (segment (start 170.930001 120.56) (end 170.930001 118.907997) (width 0.2) (layer "F.Cu") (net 11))
 (segment (start 168.430001 120.56) (end 168.430001 121.891999) (width 0.2) (layer "F.Cu") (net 15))
 (segment (start 168.430001 121.891999) (end 168.402 121.92) (width 0.2) (layer "F.Cu") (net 15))
 (via (at 168.402 121.92) (size 0.6) (drill 0.3) (layers "F.Cu" "B.Cu") (free yes) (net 15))
 (segment (start 173.99 121.92) (end 177.8 118.11) (width 0.2) (layer "B.Cu") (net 15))
 (segment (start 168.402 121.92) (end 173.99 121.92) (width 0.2) (layer "B.Cu") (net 15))
 (segment (start 169.418 119.4054) (end 169.93 119.9174) (width 0.2) (layer "F.Cu") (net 13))
 (segment (start 169.93 119.9174) (end 169.93 120.56) (width 0.2) (layer "F.Cu") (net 13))
 (via (at 169.418 119.4054) (size 0.6) (drill 0.3) (layers "F.Cu" "B.Cu") (free yes) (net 13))
 (segment (start 171.4246 119.4054) (end 169.418 119.4054) (width 0.2) (layer "B.Cu") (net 13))
 (segment (start 177.8 113.03) (end 171.4246 119.4054) (width 0.2) (layer "B.Cu") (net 13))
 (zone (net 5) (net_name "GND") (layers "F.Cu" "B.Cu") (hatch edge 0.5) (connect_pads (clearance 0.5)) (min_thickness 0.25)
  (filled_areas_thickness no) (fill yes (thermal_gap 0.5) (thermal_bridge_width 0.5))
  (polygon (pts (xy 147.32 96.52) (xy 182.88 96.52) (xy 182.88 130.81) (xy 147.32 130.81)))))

